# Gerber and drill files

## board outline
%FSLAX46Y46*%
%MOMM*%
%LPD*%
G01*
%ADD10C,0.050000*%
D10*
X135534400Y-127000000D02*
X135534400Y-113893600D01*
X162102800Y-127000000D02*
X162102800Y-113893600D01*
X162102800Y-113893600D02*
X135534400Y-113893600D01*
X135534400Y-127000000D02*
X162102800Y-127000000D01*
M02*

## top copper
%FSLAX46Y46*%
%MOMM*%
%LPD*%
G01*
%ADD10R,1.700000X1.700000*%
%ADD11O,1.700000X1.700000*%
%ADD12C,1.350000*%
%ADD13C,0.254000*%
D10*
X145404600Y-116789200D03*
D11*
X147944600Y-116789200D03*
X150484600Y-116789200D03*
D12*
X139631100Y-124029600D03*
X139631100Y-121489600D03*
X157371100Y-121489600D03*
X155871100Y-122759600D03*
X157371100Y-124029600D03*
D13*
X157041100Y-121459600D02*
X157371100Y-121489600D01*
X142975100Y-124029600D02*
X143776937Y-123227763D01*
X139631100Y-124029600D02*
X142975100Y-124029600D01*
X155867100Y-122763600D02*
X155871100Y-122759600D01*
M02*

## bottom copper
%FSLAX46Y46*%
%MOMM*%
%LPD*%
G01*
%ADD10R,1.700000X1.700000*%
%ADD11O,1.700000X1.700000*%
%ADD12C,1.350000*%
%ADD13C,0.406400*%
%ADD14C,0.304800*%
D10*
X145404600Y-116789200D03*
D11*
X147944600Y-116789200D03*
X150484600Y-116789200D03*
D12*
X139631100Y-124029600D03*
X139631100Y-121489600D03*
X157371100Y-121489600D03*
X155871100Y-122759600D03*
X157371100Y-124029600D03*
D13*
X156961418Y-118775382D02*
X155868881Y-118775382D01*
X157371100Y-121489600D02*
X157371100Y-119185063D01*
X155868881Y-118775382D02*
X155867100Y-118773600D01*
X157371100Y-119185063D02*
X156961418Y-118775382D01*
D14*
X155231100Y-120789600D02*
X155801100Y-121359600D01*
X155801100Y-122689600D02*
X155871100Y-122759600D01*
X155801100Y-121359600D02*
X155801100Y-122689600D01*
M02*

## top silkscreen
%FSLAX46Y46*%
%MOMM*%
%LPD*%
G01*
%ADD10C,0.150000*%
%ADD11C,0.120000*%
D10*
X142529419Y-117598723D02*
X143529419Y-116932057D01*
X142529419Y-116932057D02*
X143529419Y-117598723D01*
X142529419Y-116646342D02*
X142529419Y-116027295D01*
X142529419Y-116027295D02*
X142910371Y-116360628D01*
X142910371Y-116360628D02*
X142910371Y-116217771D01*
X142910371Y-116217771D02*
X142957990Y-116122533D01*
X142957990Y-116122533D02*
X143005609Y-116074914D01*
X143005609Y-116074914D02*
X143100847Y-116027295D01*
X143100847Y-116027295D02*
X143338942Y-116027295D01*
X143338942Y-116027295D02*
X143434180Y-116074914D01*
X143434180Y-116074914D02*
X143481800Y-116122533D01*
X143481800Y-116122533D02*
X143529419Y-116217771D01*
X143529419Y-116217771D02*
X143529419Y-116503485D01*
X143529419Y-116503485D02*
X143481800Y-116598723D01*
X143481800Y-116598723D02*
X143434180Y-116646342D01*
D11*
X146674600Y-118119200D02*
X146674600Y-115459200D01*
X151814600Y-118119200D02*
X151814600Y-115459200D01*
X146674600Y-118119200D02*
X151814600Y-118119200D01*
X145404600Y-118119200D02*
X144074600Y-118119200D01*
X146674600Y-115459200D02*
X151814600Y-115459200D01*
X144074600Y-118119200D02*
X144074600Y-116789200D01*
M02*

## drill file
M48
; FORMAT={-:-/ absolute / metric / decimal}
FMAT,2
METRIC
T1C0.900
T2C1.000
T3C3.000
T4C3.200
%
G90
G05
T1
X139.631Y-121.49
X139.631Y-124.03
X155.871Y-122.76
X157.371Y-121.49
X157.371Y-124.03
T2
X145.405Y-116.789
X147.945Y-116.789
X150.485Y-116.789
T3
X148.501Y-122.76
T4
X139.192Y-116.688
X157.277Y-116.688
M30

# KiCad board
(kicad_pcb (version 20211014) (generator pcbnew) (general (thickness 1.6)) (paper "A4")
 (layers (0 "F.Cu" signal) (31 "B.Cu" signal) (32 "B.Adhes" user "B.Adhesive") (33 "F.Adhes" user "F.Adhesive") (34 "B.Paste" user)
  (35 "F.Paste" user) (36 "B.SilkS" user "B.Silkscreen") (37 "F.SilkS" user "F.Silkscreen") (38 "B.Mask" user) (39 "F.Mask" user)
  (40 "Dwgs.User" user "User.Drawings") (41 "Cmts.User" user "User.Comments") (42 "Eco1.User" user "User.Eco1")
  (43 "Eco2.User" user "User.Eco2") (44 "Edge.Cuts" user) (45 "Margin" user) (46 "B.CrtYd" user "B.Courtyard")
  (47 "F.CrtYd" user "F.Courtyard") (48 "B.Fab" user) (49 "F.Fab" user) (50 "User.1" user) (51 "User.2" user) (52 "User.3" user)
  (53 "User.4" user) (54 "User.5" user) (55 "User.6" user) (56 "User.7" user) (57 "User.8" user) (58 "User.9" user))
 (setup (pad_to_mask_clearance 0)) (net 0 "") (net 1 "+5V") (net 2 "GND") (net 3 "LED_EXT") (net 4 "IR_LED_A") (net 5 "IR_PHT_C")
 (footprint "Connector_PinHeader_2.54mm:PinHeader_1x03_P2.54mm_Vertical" (layer "F.Cu") (at 145.4046 116.7892 90)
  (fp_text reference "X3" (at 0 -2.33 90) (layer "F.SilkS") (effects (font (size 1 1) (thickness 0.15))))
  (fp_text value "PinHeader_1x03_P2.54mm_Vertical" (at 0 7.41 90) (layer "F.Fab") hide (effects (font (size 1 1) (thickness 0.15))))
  (fp_line (start -1.33 1.27) (end 1.33 1.27) (layer "F.SilkS") (width 0.12))
  (fp_line (start -1.33 6.41) (end 1.33 6.41) (layer "F.SilkS") (width 0.12))
  (fp_line (start -1.33 1.27) (end -1.33 6.41) (layer "F.SilkS") (width 0.12))
  (fp_line (start -1.33 0) (end -1.33 -1.33) (layer "F.SilkS") (width 0.12))
  (fp_line (start 1.33 1.27) (end 1.33 6.41) (layer "F.SilkS") (width 0.12))
  (fp_line (start -1.33 -1.33) (end 0 -1.33) (layer "F.SilkS") (width 0.12))
  (pad "1" thru_hole rect (at 0 0 90) (size 1.7 1.7) (drill 1) (layers *.Cu *.Mask) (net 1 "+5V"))
  (pad "2" thru_hole oval (at 0 2.54 90) (size 1.7 1.7) (drill 1) (layers *.Cu *.Mask) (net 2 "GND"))
  (pad "3" thru_hole oval (at 0 5.08 90) (size 1.7 1.7) (drill 1) (layers *.Cu *.Mask) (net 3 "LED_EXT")))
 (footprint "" (layer "F.Cu") (at 148.5011 122.7596)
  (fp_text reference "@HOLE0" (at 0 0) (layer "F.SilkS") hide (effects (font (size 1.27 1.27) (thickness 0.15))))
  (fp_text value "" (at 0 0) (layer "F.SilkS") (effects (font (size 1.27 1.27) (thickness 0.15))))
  (pad "" np_thru_hole circle (at 0 0) (size 3 3) (drill 3) (layers *.Cu *.Mask)))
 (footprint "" (layer "F.Cu") (at 139.192 116.6876)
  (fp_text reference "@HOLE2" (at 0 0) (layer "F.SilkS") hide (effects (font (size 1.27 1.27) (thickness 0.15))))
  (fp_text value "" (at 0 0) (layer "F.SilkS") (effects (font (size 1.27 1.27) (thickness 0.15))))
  (pad "" np_thru_hole circle (at 0 0) (size 3.2 3.2) (drill 3.2) (layers *.Cu *.Mask)))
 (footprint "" (layer "F.Cu") (at 157.2768 116.6876)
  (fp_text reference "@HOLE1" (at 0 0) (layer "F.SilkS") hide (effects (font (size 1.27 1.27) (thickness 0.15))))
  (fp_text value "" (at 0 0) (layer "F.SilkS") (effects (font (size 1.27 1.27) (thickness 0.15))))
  (pad "" np_thru_hole circle (at 0 0) (size 3.2 3.2) (drill 3.2) (layers *.Cu *.Mask)))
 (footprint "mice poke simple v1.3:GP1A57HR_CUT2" (layer "B.Cu") (at 148.5011 122.7596 -90)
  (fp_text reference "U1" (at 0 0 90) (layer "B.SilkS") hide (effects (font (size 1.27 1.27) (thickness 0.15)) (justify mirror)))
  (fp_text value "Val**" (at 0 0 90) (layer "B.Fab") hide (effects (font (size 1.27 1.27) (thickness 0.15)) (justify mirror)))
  (pad "1" thru_hole circle (at 1.27 8.87 270) (size 1.35 1.35) (drill 0.9) (layers *.Cu *.Mask) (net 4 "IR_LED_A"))
  (pad "2" thru_hole circle (at -1.27 8.87 270) (size 1.35 1.35) (drill 0.9) (layers *.Cu *.Mask) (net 2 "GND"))
  (pad "3" thru_hole circle (at -1.27 -8.87 270) (size 1.35 1.35) (drill 0.9) (layers *.Cu *.Mask) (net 1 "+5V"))
  (pad "4" thru_hole circle (at 0 -7.37 270) (size 1.35 1.35) (drill 0.9) (layers *.Cu *.Mask) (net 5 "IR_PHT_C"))
  (pad "5" thru_hole circle (at 1.27 -8.87 270) (size 1.35 1.35) (drill 0.9) (layers *.Cu *.Mask) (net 2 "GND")))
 (gr_line (start 135.5344 127) (end 135.5344 113.8936) (layer "Edge.Cuts") (width 0.05))
 (gr_line (start 162.1028 127) (end 162.1028 113.8936) (layer "Edge.Cuts") (width 0.05))
 (gr_line (start 162.1028 113.8936) (end 135.5344 113.8936) (layer "Edge.Cuts") (width 0.05))
 (gr_line (start 135.5344 127) (end 162.1028 127) (layer "Edge.Cuts") (width 0.05))
 (segment (start 157.0411 121.4596) (end 157.3711 121.4896) (width 0.254) (layer "F.Cu") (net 1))
 (segment (start 156.961418 118.775382) (end 155.868881 118.775382) (width 0.4064) (layer "B.Cu") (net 1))
 (segment (start 157.3711 121.4896) (end 157.3711 119.185063) (width 0.4064) (layer "B.Cu") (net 1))
 (segment (start 155.868881 118.775382) (end 155.8671 118.7736) (width 0.4064) (layer "B.Cu") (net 1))
 (segment (start 157.3711 119.185063) (end 156.961418 118.775382) (width 0.4064) (layer "B.Cu") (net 1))
 (segment (start 142.9751 124.0296) (end 143.776937 123.227763) (width 0.254) (layer "F.Cu") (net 4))
 (segment (start 139.6311 124.0296) (end 142.9751 124.0296) (width 0.254) (layer "F.Cu") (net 4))
 (segment (start 155.8671 122.7636) (end 155.8711 122.7596) (width 0.254) (layer "F.Cu") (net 5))
 (segment (start 155.2311 120.7896) (end 155.8011 121.3596) (width 0.3048) (layer "B.Cu") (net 5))
 (segment (start 155.8011 122.6896) (end 155.8711 122.7596) (width 0.3048) (layer "B.Cu") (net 5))
 (segment (start 155.8011 121.3596) (end 155.8011 122.6896) (width 0.3048) (layer "B.Cu") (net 5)))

